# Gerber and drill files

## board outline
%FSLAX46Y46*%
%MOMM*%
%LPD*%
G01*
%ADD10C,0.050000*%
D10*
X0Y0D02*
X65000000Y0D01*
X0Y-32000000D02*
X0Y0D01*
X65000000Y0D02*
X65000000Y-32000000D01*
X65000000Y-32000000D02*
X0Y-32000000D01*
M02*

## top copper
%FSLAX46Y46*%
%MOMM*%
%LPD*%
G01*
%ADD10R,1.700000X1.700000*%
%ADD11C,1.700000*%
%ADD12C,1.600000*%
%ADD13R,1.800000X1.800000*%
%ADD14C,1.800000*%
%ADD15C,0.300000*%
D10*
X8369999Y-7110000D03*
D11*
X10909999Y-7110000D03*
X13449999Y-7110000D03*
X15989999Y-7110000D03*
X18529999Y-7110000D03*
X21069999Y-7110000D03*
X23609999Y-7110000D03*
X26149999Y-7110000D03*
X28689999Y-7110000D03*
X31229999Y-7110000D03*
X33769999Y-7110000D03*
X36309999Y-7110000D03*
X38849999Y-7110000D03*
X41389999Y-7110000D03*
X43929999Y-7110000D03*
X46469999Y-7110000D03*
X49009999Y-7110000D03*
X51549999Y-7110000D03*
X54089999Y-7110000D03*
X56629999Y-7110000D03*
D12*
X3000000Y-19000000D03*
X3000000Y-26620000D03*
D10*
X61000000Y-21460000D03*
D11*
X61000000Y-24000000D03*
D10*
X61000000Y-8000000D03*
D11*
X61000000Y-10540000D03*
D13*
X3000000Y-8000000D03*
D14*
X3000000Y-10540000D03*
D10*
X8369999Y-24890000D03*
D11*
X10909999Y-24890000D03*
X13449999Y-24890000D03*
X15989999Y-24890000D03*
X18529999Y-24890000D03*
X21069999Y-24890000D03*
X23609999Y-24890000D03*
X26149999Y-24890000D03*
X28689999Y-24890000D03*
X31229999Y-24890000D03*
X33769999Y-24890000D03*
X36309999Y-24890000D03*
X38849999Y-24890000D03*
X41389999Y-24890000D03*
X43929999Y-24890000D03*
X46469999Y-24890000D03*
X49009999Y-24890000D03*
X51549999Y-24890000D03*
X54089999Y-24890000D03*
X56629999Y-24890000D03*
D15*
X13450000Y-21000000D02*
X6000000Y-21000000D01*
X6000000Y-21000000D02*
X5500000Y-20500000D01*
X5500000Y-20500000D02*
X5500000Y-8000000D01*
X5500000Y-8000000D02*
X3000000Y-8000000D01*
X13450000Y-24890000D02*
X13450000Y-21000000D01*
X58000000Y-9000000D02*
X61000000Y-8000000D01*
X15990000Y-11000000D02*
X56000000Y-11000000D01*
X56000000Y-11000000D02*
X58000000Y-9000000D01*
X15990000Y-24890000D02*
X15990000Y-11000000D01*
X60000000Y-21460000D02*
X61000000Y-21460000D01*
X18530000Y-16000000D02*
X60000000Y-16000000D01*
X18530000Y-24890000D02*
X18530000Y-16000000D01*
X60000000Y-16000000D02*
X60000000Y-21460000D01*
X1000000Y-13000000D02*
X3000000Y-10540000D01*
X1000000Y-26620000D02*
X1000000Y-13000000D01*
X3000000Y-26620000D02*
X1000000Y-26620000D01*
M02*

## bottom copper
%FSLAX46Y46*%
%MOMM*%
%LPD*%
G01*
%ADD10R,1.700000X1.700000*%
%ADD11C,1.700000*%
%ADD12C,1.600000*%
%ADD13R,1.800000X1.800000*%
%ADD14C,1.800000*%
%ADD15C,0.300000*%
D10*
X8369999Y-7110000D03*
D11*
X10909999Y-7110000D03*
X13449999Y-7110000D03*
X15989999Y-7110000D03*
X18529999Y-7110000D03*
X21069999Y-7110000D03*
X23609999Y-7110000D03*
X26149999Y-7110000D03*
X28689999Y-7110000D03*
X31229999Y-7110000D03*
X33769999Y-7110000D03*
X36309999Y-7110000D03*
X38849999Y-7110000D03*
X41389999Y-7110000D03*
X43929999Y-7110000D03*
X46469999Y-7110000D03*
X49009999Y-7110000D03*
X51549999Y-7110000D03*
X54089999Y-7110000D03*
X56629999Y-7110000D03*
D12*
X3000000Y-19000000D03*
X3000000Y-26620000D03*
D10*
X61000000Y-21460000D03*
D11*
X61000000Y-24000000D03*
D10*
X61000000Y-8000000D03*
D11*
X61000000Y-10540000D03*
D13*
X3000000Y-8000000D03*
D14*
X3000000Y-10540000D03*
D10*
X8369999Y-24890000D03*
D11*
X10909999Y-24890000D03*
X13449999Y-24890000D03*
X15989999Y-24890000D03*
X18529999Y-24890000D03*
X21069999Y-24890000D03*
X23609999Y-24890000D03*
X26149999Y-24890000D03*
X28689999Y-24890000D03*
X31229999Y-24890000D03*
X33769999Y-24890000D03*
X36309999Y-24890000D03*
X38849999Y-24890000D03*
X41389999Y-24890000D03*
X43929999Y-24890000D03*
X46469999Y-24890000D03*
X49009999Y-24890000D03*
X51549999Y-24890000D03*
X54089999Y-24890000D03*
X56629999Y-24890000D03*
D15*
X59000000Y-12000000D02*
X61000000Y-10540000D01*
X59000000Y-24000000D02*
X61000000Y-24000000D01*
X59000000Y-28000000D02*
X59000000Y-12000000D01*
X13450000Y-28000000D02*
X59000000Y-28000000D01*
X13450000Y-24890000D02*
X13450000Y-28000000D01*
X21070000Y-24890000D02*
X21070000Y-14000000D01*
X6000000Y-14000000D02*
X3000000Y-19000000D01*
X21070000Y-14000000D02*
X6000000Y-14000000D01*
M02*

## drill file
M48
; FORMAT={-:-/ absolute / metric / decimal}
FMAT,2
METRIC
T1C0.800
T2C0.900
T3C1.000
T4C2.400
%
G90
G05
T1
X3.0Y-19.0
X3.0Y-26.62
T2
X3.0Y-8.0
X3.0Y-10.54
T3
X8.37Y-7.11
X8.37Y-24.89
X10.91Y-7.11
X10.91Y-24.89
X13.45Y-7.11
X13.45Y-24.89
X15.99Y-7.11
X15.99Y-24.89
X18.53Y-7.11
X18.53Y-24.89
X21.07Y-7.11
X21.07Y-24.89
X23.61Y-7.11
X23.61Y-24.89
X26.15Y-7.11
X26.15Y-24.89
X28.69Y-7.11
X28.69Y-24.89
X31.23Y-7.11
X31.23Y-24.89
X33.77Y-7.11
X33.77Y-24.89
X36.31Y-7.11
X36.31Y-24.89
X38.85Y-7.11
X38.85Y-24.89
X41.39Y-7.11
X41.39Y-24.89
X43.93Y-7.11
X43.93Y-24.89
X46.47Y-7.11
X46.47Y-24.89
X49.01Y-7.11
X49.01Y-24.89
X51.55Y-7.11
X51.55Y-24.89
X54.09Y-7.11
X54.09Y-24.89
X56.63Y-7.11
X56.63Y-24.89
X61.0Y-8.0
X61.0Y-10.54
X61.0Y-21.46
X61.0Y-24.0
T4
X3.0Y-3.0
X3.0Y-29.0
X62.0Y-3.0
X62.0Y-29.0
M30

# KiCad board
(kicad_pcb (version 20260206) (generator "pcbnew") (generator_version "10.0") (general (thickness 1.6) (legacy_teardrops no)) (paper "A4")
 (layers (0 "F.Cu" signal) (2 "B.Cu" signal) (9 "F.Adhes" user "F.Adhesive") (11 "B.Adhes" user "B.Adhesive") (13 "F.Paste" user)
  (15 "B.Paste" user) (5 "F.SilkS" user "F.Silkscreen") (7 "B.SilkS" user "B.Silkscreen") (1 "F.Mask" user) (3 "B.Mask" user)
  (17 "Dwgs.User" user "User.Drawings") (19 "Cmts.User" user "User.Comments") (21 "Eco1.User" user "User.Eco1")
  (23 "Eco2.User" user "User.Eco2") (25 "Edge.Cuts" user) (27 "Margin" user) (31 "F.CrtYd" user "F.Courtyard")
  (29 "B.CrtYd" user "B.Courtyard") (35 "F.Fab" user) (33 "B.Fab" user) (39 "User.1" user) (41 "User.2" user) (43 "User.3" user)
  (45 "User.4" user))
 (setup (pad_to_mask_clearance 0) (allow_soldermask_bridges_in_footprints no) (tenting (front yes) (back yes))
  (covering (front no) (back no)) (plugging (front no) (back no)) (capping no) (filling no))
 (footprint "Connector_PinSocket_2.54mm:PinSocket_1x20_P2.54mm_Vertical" (layer "F.Cu") (at 8.369999 7.11 90)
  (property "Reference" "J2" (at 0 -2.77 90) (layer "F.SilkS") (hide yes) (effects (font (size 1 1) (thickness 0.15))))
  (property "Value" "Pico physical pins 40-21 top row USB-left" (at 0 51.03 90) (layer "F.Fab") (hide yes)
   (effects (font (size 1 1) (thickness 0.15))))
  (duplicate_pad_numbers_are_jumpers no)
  (pad "1" thru_hole rect (at 0 0 90) (size 1.7 1.7) (drill 1) (layers "*.Cu" "*.Mask") (remove_unused_layers no)
   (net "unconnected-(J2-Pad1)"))
  (pad "2" thru_hole circle (at 0 2.54 90) (size 1.7 1.7) (drill 1) (layers "*.Cu" "*.Mask") (remove_unused_layers no)
   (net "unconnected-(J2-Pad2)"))
  (pad "3" thru_hole circle (at 0 5.08 90) (size 1.7 1.7) (drill 1) (layers "*.Cu" "*.Mask") (remove_unused_layers no)
   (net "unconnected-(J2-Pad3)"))
  (pad "4" thru_hole circle (at 0 7.62 90) (size 1.7 1.7) (drill 1) (layers "*.Cu" "*.Mask") (remove_unused_layers no)
   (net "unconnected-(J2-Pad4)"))
  (pad "5" thru_hole circle (at 0 10.16 90) (size 1.7 1.7) (drill 1) (layers "*.Cu" "*.Mask") (remove_unused_layers no)
   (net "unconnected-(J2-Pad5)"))
  (pad "6" thru_hole circle (at 0 12.7 90) (size 1.7 1.7) (drill 1) (layers "*.Cu" "*.Mask") (remove_unused_layers no)
   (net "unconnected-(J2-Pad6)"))
  (pad "7" thru_hole circle (at 0 15.24 90) (size 1.7 1.7) (drill 1) (layers "*.Cu" "*.Mask") (remove_unused_layers no)
   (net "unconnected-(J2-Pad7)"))
  (pad "8" thru_hole circle (at 0 17.78 90) (size 1.7 1.7) (drill 1) (layers "*.Cu" "*.Mask") (remove_unused_layers no)
   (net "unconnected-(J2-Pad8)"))
  (pad "9" thru_hole circle (at 0 20.32 90) (size 1.7 1.7) (drill 1) (layers "*.Cu" "*.Mask") (remove_unused_layers no)
   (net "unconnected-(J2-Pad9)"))
  (pad "10" thru_hole circle (at 0 22.86 90) (size 1.7 1.7) (drill 1) (layers "*.Cu" "*.Mask") (remove_unused_layers no)
   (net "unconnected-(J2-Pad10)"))
  (pad "11" thru_hole circle (at 0 25.4 90) (size 1.7 1.7) (drill 1) (layers "*.Cu" "*.Mask") (remove_unused_layers no)
   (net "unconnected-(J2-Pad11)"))
  (pad "12" thru_hole circle (at 0 27.94 90) (size 1.7 1.7) (drill 1) (layers "*.Cu" "*.Mask") (remove_unused_layers no)
   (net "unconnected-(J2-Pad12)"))
  (pad "13" thru_hole circle (at 0 30.48 90) (size 1.7 1.7) (drill 1) (layers "*.Cu" "*.Mask") (remove_unused_layers no)
   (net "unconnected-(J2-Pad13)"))
  (pad "14" thru_hole circle (at 0 33.02 90) (size 1.7 1.7) (drill 1) (layers "*.Cu" "*.Mask") (remove_unused_layers no)
   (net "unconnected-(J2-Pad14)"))
  (pad "15" thru_hole circle (at 0 35.56 90) (size 1.7 1.7) (drill 1) (layers "*.Cu" "*.Mask") (remove_unused_layers no)
   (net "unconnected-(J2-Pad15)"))
  (pad "16" thru_hole circle (at 0 38.1 90) (size 1.7 1.7) (drill 1) (layers "*.Cu" "*.Mask") (remove_unused_layers no)
   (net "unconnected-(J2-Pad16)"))
  (pad "17" thru_hole circle (at 0 40.64 90) (size 1.7 1.7) (drill 1) (layers "*.Cu" "*.Mask") (remove_unused_layers no)
   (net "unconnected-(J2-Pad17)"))
  (pad "18" thru_hole circle (at 0 43.18 90) (size 1.7 1.7) (drill 1) (layers "*.Cu" "*.Mask") (remove_unused_layers no)
   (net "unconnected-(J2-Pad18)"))
  (pad "19" thru_hole circle (at 0 45.72 90) (size 1.7 1.7) (drill 1) (layers "*.Cu" "*.Mask") (remove_unused_layers no)
   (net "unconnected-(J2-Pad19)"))
  (pad "20" thru_hole circle (at 0 48.26 90) (size 1.7 1.7) (drill 1) (layers "*.Cu" "*.Mask") (remove_unused_layers no)
   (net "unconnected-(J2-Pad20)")))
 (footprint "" (layer "F.Cu") (at 3 29)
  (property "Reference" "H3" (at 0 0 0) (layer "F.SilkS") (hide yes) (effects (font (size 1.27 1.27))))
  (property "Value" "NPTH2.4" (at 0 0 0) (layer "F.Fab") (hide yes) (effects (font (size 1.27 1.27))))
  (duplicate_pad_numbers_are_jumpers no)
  (pad "" np_thru_hole circle (at 0 0) (size 2.4 2.4) (drill 2.4) (layers "*.Cu")))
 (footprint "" (layer "F.Cu") (at 62 29)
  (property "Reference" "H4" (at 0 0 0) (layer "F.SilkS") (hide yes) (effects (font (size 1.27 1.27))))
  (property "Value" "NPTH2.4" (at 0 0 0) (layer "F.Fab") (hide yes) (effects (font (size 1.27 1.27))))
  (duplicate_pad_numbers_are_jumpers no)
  (pad "" np_thru_hole circle (at 0 0) (size 2.4 2.4) (drill 2.4) (layers "*.Cu")))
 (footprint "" (layer "F.Cu") (at 3 3)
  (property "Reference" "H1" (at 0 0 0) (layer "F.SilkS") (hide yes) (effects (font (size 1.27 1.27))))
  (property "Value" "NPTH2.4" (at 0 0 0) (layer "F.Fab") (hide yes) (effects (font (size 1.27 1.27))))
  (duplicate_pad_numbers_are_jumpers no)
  (pad "" np_thru_hole circle (at 0 0) (size 2.4 2.4) (drill 2.4) (layers "*.Cu")))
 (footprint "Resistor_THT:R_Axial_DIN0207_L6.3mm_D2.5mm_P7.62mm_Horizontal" (layer "F.Cu") (at 3 19 -90)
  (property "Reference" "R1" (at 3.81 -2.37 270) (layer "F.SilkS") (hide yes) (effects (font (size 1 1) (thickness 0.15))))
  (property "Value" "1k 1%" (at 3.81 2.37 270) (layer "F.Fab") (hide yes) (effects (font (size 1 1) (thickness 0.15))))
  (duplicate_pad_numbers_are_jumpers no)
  (pad "1" thru_hole circle (at 0 0 270) (size 1.6 1.6) (drill 0.8) (layers "*.Cu" "*.Mask") (remove_unused_layers no) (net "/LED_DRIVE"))
  (pad "2" thru_hole circle (at 7.62 0 270) (size 1.6 1.6) (drill 0.8) (layers "*.Cu" "*.Mask") (remove_unused_layers no) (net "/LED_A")))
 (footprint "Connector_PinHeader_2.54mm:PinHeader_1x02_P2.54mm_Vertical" (layer "F.Cu") (at 61 21.46)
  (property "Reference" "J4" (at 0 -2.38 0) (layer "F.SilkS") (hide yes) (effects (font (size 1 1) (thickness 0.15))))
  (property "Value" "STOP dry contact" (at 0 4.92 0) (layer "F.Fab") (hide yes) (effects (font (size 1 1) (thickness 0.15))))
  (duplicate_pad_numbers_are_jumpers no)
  (pad "1" thru_hole rect (at 0 0) (size 1.7 1.7) (drill 1) (layers "*.Cu" "*.Mask") (remove_unused_layers no) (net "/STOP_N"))
  (pad "2" thru_hole circle (at 0 2.54) (size 1.7 1.7) (drill 1) (layers "*.Cu" "*.Mask") (remove_unused_layers no) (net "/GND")))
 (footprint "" (layer "F.Cu") (at 62 3)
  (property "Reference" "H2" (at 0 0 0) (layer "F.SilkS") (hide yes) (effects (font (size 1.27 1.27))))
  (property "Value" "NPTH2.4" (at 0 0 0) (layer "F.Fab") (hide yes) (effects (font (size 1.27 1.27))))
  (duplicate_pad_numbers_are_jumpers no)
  (pad "" np_thru_hole circle (at 0 0) (size 2.4 2.4) (drill 2.4) (layers "*.Cu")))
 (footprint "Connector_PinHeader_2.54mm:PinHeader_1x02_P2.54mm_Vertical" (layer "F.Cu") (at 61 8)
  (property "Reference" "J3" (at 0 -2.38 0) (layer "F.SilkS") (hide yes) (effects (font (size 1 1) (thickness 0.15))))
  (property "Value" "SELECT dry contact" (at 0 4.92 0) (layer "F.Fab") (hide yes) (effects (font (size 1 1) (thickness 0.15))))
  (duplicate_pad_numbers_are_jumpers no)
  (pad "1" thru_hole rect (at 0 0) (size 1.7 1.7) (drill 1) (layers "*.Cu" "*.Mask") (remove_unused_layers no) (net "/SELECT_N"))
  (pad "2" thru_hole circle (at 0 2.54) (size 1.7 1.7) (drill 1) (layers "*.Cu" "*.Mask") (remove_unused_layers no) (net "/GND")))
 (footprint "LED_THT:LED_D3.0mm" (layer "F.Cu") (at 3 8 -90)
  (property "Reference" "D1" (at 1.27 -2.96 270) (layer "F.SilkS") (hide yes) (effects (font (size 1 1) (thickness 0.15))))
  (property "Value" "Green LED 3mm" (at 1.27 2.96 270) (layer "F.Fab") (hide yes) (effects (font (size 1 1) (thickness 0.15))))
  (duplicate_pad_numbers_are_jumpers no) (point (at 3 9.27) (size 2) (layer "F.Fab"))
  (pad "1" thru_hole rect (at 0 0 270) (size 1.8 1.8) (drill 0.9) (layers "*.Cu" "*.Mask") (remove_unused_layers no) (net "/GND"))
  (pad "2" thru_hole circle (at 2.54 0 270) (size 1.8 1.8) (drill 0.9) (layers "*.Cu" "*.Mask") (remove_unused_layers no) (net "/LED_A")))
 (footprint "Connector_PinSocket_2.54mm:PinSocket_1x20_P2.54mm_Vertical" (layer "F.Cu") (at 8.369999 24.89 90)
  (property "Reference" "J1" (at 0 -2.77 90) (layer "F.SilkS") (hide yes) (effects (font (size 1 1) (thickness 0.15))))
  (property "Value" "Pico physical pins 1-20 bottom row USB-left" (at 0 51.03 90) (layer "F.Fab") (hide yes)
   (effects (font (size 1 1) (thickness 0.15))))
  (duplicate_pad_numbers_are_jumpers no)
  (pad "1" thru_hole rect (at 0 0 90) (size 1.7 1.7) (drill 1) (layers "*.Cu" "*.Mask") (remove_unused_layers no)
   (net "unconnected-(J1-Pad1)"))
  (pad "2" thru_hole circle (at 0 2.54 90) (size 1.7 1.7) (drill 1) (layers "*.Cu" "*.Mask") (remove_unused_layers no)
   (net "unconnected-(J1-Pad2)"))
  (pad "3" thru_hole circle (at 0 5.08 90) (size 1.7 1.7) (drill 1) (layers "*.Cu" "*.Mask") (remove_unused_layers no) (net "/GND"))
  (pad "4" thru_hole circle (at 0 7.62 90) (size 1.7 1.7) (drill 1) (layers "*.Cu" "*.Mask") (remove_unused_layers no) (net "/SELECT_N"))
  (pad "5" thru_hole circle (at 0 10.16 90) (size 1.7 1.7) (drill 1) (layers "*.Cu" "*.Mask") (remove_unused_layers no) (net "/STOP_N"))
  (pad "6" thru_hole circle (at 0 12.7 90) (size 1.7 1.7) (drill 1) (layers "*.Cu" "*.Mask") (remove_unused_layers no) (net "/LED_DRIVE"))
  (pad "7" thru_hole circle (at 0 15.24 90) (size 1.7 1.7) (drill 1) (layers "*.Cu" "*.Mask") (remove_unused_layers no)
   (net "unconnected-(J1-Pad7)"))
  (pad "8" thru_hole circle (at 0 17.78 90) (size 1.7 1.7) (drill 1) (layers "*.Cu" "*.Mask") (remove_unused_layers no)
   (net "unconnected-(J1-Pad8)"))
  (pad "9" thru_hole circle (at 0 20.32 90) (size 1.7 1.7) (drill 1) (layers "*.Cu" "*.Mask") (remove_unused_layers no)
   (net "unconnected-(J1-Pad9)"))
  (pad "10" thru_hole circle (at 0 22.86 90) (size 1.7 1.7) (drill 1) (layers "*.Cu" "*.Mask") (remove_unused_layers no)
   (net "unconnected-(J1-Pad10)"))
  (pad "11" thru_hole circle (at 0 25.4 90) (size 1.7 1.7) (drill 1) (layers "*.Cu" "*.Mask") (remove_unused_layers no)
   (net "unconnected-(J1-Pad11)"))
  (pad "12" thru_hole circle (at 0 27.94 90) (size 1.7 1.7) (drill 1) (layers "*.Cu" "*.Mask") (remove_unused_layers no)
   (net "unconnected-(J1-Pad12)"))
  (pad "13" thru_hole circle (at 0 30.48 90) (size 1.7 1.7) (drill 1) (layers "*.Cu" "*.Mask") (remove_unused_layers no)
   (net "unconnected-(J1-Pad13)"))
  (pad "14" thru_hole circle (at 0 33.02 90) (size 1.7 1.7) (drill 1) (layers "*.Cu" "*.Mask") (remove_unused_layers no)
   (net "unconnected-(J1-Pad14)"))
  (pad "15" thru_hole circle (at 0 35.56 90) (size 1.7 1.7) (drill 1) (layers "*.Cu" "*.Mask") (remove_unused_layers no)
   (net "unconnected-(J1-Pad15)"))
  (pad "16" thru_hole circle (at 0 38.1 90) (size 1.7 1.7) (drill 1) (layers "*.Cu" "*.Mask") (remove_unused_layers no)
   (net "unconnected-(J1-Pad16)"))
  (pad "17" thru_hole circle (at 0 40.64 90) (size 1.7 1.7) (drill 1) (layers "*.Cu" "*.Mask") (remove_unused_layers no)
   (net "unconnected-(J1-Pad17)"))
  (pad "18" thru_hole circle (at 0 43.18 90) (size 1.7 1.7) (drill 1) (layers "*.Cu" "*.Mask") (remove_unused_layers no)
   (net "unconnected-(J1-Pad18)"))
  (pad "19" thru_hole circle (at 0 45.72 90) (size 1.7 1.7) (drill 1) (layers "*.Cu" "*.Mask") (remove_unused_layers no)
   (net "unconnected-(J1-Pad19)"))
  (pad "20" thru_hole circle (at 0 48.26 90) (size 1.7 1.7) (drill 1) (layers "*.Cu" "*.Mask") (remove_unused_layers no)
   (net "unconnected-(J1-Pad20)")))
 (gr_line (start 0 0) (end 65 0) (stroke (width 0.05) (type default)) (layer "Edge.Cuts"))
 (gr_line (start 0 32) (end 0 0) (stroke (width 0.05) (type default)) (layer "Edge.Cuts"))
 (gr_line (start 65 0) (end 65 32) (stroke (width 0.05) (type default)) (layer "Edge.Cuts"))
 (gr_line (start 65 32) (end 0 32) (stroke (width 0.05) (type default)) (layer "Edge.Cuts"))
 (segment (start 13.45 21) (end 6 21) (width 0.3) (layer "F.Cu") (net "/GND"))
 (segment (start 6 21) (end 5.5 20.5) (width 0.3) (layer "F.Cu") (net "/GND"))
 (segment (start 5.5 20.5) (end 5.5 8) (width 0.3) (layer "F.Cu") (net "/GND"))
 (segment (start 5.5 8) (end 3 8) (width 0.3) (layer "F.Cu") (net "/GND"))
 (segment (start 13.45 24.89) (end 13.45 21) (width 0.3) (layer "F.Cu") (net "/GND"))
 (segment (start 59 12) (end 61 10.54) (width 0.3) (layer "B.Cu") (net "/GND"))
 (segment (start 59 24) (end 61 24) (width 0.3) (layer "B.Cu") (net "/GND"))
 (segment (start 59 28) (end 59 12) (width 0.3) (layer "B.Cu") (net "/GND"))
 (segment (start 13.45 28) (end 59 28) (width 0.3) (layer "B.Cu") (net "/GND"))
 (segment (start 13.45 24.89) (end 13.45 28) (width 0.3) (layer "B.Cu") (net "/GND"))
 (segment (start 58 9) (end 61 8) (width 0.3) (layer "F.Cu") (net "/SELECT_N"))
 (segment (start 15.99 11) (end 56 11) (width 0.3) (layer "F.Cu") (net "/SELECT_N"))
 (segment (start 56 11) (end 58 9) (width 0.3) (layer "F.Cu") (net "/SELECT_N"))
 (segment (start 15.99 24.89) (end 15.99 11) (width 0.3) (layer "F.Cu") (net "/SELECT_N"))
 (segment (start 60 21.46) (end 61 21.46) (width 0.3) (layer "F.Cu") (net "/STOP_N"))
 (segment (start 18.53 16) (end 60 16) (width 0.3) (layer "F.Cu") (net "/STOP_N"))
 (segment (start 18.53 24.89) (end 18.53 16) (width 0.3) (layer "F.Cu") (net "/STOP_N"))
 (segment (start 60 16) (end 60 21.46) (width 0.3) (layer "F.Cu") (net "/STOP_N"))
 (segment (start 21.07 24.89) (end 21.07 14) (width 0.3) (layer "B.Cu") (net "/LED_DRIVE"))
 (segment (start 6 14) (end 3 19) (width 0.3) (layer "B.Cu") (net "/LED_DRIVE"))
 (segment (start 21.07 14) (end 6 14) (width 0.3) (layer "B.Cu") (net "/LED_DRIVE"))
 (segment (start 1 13) (end 3 10.54) (width 0.3) (layer "F.Cu") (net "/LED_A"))
 (segment (start 1 26.62) (end 1 13) (width 0.3) (layer "F.Cu") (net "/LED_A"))
 (segment (start 3 26.62) (end 1 26.62) (width 0.3) (layer "F.Cu") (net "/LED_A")))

